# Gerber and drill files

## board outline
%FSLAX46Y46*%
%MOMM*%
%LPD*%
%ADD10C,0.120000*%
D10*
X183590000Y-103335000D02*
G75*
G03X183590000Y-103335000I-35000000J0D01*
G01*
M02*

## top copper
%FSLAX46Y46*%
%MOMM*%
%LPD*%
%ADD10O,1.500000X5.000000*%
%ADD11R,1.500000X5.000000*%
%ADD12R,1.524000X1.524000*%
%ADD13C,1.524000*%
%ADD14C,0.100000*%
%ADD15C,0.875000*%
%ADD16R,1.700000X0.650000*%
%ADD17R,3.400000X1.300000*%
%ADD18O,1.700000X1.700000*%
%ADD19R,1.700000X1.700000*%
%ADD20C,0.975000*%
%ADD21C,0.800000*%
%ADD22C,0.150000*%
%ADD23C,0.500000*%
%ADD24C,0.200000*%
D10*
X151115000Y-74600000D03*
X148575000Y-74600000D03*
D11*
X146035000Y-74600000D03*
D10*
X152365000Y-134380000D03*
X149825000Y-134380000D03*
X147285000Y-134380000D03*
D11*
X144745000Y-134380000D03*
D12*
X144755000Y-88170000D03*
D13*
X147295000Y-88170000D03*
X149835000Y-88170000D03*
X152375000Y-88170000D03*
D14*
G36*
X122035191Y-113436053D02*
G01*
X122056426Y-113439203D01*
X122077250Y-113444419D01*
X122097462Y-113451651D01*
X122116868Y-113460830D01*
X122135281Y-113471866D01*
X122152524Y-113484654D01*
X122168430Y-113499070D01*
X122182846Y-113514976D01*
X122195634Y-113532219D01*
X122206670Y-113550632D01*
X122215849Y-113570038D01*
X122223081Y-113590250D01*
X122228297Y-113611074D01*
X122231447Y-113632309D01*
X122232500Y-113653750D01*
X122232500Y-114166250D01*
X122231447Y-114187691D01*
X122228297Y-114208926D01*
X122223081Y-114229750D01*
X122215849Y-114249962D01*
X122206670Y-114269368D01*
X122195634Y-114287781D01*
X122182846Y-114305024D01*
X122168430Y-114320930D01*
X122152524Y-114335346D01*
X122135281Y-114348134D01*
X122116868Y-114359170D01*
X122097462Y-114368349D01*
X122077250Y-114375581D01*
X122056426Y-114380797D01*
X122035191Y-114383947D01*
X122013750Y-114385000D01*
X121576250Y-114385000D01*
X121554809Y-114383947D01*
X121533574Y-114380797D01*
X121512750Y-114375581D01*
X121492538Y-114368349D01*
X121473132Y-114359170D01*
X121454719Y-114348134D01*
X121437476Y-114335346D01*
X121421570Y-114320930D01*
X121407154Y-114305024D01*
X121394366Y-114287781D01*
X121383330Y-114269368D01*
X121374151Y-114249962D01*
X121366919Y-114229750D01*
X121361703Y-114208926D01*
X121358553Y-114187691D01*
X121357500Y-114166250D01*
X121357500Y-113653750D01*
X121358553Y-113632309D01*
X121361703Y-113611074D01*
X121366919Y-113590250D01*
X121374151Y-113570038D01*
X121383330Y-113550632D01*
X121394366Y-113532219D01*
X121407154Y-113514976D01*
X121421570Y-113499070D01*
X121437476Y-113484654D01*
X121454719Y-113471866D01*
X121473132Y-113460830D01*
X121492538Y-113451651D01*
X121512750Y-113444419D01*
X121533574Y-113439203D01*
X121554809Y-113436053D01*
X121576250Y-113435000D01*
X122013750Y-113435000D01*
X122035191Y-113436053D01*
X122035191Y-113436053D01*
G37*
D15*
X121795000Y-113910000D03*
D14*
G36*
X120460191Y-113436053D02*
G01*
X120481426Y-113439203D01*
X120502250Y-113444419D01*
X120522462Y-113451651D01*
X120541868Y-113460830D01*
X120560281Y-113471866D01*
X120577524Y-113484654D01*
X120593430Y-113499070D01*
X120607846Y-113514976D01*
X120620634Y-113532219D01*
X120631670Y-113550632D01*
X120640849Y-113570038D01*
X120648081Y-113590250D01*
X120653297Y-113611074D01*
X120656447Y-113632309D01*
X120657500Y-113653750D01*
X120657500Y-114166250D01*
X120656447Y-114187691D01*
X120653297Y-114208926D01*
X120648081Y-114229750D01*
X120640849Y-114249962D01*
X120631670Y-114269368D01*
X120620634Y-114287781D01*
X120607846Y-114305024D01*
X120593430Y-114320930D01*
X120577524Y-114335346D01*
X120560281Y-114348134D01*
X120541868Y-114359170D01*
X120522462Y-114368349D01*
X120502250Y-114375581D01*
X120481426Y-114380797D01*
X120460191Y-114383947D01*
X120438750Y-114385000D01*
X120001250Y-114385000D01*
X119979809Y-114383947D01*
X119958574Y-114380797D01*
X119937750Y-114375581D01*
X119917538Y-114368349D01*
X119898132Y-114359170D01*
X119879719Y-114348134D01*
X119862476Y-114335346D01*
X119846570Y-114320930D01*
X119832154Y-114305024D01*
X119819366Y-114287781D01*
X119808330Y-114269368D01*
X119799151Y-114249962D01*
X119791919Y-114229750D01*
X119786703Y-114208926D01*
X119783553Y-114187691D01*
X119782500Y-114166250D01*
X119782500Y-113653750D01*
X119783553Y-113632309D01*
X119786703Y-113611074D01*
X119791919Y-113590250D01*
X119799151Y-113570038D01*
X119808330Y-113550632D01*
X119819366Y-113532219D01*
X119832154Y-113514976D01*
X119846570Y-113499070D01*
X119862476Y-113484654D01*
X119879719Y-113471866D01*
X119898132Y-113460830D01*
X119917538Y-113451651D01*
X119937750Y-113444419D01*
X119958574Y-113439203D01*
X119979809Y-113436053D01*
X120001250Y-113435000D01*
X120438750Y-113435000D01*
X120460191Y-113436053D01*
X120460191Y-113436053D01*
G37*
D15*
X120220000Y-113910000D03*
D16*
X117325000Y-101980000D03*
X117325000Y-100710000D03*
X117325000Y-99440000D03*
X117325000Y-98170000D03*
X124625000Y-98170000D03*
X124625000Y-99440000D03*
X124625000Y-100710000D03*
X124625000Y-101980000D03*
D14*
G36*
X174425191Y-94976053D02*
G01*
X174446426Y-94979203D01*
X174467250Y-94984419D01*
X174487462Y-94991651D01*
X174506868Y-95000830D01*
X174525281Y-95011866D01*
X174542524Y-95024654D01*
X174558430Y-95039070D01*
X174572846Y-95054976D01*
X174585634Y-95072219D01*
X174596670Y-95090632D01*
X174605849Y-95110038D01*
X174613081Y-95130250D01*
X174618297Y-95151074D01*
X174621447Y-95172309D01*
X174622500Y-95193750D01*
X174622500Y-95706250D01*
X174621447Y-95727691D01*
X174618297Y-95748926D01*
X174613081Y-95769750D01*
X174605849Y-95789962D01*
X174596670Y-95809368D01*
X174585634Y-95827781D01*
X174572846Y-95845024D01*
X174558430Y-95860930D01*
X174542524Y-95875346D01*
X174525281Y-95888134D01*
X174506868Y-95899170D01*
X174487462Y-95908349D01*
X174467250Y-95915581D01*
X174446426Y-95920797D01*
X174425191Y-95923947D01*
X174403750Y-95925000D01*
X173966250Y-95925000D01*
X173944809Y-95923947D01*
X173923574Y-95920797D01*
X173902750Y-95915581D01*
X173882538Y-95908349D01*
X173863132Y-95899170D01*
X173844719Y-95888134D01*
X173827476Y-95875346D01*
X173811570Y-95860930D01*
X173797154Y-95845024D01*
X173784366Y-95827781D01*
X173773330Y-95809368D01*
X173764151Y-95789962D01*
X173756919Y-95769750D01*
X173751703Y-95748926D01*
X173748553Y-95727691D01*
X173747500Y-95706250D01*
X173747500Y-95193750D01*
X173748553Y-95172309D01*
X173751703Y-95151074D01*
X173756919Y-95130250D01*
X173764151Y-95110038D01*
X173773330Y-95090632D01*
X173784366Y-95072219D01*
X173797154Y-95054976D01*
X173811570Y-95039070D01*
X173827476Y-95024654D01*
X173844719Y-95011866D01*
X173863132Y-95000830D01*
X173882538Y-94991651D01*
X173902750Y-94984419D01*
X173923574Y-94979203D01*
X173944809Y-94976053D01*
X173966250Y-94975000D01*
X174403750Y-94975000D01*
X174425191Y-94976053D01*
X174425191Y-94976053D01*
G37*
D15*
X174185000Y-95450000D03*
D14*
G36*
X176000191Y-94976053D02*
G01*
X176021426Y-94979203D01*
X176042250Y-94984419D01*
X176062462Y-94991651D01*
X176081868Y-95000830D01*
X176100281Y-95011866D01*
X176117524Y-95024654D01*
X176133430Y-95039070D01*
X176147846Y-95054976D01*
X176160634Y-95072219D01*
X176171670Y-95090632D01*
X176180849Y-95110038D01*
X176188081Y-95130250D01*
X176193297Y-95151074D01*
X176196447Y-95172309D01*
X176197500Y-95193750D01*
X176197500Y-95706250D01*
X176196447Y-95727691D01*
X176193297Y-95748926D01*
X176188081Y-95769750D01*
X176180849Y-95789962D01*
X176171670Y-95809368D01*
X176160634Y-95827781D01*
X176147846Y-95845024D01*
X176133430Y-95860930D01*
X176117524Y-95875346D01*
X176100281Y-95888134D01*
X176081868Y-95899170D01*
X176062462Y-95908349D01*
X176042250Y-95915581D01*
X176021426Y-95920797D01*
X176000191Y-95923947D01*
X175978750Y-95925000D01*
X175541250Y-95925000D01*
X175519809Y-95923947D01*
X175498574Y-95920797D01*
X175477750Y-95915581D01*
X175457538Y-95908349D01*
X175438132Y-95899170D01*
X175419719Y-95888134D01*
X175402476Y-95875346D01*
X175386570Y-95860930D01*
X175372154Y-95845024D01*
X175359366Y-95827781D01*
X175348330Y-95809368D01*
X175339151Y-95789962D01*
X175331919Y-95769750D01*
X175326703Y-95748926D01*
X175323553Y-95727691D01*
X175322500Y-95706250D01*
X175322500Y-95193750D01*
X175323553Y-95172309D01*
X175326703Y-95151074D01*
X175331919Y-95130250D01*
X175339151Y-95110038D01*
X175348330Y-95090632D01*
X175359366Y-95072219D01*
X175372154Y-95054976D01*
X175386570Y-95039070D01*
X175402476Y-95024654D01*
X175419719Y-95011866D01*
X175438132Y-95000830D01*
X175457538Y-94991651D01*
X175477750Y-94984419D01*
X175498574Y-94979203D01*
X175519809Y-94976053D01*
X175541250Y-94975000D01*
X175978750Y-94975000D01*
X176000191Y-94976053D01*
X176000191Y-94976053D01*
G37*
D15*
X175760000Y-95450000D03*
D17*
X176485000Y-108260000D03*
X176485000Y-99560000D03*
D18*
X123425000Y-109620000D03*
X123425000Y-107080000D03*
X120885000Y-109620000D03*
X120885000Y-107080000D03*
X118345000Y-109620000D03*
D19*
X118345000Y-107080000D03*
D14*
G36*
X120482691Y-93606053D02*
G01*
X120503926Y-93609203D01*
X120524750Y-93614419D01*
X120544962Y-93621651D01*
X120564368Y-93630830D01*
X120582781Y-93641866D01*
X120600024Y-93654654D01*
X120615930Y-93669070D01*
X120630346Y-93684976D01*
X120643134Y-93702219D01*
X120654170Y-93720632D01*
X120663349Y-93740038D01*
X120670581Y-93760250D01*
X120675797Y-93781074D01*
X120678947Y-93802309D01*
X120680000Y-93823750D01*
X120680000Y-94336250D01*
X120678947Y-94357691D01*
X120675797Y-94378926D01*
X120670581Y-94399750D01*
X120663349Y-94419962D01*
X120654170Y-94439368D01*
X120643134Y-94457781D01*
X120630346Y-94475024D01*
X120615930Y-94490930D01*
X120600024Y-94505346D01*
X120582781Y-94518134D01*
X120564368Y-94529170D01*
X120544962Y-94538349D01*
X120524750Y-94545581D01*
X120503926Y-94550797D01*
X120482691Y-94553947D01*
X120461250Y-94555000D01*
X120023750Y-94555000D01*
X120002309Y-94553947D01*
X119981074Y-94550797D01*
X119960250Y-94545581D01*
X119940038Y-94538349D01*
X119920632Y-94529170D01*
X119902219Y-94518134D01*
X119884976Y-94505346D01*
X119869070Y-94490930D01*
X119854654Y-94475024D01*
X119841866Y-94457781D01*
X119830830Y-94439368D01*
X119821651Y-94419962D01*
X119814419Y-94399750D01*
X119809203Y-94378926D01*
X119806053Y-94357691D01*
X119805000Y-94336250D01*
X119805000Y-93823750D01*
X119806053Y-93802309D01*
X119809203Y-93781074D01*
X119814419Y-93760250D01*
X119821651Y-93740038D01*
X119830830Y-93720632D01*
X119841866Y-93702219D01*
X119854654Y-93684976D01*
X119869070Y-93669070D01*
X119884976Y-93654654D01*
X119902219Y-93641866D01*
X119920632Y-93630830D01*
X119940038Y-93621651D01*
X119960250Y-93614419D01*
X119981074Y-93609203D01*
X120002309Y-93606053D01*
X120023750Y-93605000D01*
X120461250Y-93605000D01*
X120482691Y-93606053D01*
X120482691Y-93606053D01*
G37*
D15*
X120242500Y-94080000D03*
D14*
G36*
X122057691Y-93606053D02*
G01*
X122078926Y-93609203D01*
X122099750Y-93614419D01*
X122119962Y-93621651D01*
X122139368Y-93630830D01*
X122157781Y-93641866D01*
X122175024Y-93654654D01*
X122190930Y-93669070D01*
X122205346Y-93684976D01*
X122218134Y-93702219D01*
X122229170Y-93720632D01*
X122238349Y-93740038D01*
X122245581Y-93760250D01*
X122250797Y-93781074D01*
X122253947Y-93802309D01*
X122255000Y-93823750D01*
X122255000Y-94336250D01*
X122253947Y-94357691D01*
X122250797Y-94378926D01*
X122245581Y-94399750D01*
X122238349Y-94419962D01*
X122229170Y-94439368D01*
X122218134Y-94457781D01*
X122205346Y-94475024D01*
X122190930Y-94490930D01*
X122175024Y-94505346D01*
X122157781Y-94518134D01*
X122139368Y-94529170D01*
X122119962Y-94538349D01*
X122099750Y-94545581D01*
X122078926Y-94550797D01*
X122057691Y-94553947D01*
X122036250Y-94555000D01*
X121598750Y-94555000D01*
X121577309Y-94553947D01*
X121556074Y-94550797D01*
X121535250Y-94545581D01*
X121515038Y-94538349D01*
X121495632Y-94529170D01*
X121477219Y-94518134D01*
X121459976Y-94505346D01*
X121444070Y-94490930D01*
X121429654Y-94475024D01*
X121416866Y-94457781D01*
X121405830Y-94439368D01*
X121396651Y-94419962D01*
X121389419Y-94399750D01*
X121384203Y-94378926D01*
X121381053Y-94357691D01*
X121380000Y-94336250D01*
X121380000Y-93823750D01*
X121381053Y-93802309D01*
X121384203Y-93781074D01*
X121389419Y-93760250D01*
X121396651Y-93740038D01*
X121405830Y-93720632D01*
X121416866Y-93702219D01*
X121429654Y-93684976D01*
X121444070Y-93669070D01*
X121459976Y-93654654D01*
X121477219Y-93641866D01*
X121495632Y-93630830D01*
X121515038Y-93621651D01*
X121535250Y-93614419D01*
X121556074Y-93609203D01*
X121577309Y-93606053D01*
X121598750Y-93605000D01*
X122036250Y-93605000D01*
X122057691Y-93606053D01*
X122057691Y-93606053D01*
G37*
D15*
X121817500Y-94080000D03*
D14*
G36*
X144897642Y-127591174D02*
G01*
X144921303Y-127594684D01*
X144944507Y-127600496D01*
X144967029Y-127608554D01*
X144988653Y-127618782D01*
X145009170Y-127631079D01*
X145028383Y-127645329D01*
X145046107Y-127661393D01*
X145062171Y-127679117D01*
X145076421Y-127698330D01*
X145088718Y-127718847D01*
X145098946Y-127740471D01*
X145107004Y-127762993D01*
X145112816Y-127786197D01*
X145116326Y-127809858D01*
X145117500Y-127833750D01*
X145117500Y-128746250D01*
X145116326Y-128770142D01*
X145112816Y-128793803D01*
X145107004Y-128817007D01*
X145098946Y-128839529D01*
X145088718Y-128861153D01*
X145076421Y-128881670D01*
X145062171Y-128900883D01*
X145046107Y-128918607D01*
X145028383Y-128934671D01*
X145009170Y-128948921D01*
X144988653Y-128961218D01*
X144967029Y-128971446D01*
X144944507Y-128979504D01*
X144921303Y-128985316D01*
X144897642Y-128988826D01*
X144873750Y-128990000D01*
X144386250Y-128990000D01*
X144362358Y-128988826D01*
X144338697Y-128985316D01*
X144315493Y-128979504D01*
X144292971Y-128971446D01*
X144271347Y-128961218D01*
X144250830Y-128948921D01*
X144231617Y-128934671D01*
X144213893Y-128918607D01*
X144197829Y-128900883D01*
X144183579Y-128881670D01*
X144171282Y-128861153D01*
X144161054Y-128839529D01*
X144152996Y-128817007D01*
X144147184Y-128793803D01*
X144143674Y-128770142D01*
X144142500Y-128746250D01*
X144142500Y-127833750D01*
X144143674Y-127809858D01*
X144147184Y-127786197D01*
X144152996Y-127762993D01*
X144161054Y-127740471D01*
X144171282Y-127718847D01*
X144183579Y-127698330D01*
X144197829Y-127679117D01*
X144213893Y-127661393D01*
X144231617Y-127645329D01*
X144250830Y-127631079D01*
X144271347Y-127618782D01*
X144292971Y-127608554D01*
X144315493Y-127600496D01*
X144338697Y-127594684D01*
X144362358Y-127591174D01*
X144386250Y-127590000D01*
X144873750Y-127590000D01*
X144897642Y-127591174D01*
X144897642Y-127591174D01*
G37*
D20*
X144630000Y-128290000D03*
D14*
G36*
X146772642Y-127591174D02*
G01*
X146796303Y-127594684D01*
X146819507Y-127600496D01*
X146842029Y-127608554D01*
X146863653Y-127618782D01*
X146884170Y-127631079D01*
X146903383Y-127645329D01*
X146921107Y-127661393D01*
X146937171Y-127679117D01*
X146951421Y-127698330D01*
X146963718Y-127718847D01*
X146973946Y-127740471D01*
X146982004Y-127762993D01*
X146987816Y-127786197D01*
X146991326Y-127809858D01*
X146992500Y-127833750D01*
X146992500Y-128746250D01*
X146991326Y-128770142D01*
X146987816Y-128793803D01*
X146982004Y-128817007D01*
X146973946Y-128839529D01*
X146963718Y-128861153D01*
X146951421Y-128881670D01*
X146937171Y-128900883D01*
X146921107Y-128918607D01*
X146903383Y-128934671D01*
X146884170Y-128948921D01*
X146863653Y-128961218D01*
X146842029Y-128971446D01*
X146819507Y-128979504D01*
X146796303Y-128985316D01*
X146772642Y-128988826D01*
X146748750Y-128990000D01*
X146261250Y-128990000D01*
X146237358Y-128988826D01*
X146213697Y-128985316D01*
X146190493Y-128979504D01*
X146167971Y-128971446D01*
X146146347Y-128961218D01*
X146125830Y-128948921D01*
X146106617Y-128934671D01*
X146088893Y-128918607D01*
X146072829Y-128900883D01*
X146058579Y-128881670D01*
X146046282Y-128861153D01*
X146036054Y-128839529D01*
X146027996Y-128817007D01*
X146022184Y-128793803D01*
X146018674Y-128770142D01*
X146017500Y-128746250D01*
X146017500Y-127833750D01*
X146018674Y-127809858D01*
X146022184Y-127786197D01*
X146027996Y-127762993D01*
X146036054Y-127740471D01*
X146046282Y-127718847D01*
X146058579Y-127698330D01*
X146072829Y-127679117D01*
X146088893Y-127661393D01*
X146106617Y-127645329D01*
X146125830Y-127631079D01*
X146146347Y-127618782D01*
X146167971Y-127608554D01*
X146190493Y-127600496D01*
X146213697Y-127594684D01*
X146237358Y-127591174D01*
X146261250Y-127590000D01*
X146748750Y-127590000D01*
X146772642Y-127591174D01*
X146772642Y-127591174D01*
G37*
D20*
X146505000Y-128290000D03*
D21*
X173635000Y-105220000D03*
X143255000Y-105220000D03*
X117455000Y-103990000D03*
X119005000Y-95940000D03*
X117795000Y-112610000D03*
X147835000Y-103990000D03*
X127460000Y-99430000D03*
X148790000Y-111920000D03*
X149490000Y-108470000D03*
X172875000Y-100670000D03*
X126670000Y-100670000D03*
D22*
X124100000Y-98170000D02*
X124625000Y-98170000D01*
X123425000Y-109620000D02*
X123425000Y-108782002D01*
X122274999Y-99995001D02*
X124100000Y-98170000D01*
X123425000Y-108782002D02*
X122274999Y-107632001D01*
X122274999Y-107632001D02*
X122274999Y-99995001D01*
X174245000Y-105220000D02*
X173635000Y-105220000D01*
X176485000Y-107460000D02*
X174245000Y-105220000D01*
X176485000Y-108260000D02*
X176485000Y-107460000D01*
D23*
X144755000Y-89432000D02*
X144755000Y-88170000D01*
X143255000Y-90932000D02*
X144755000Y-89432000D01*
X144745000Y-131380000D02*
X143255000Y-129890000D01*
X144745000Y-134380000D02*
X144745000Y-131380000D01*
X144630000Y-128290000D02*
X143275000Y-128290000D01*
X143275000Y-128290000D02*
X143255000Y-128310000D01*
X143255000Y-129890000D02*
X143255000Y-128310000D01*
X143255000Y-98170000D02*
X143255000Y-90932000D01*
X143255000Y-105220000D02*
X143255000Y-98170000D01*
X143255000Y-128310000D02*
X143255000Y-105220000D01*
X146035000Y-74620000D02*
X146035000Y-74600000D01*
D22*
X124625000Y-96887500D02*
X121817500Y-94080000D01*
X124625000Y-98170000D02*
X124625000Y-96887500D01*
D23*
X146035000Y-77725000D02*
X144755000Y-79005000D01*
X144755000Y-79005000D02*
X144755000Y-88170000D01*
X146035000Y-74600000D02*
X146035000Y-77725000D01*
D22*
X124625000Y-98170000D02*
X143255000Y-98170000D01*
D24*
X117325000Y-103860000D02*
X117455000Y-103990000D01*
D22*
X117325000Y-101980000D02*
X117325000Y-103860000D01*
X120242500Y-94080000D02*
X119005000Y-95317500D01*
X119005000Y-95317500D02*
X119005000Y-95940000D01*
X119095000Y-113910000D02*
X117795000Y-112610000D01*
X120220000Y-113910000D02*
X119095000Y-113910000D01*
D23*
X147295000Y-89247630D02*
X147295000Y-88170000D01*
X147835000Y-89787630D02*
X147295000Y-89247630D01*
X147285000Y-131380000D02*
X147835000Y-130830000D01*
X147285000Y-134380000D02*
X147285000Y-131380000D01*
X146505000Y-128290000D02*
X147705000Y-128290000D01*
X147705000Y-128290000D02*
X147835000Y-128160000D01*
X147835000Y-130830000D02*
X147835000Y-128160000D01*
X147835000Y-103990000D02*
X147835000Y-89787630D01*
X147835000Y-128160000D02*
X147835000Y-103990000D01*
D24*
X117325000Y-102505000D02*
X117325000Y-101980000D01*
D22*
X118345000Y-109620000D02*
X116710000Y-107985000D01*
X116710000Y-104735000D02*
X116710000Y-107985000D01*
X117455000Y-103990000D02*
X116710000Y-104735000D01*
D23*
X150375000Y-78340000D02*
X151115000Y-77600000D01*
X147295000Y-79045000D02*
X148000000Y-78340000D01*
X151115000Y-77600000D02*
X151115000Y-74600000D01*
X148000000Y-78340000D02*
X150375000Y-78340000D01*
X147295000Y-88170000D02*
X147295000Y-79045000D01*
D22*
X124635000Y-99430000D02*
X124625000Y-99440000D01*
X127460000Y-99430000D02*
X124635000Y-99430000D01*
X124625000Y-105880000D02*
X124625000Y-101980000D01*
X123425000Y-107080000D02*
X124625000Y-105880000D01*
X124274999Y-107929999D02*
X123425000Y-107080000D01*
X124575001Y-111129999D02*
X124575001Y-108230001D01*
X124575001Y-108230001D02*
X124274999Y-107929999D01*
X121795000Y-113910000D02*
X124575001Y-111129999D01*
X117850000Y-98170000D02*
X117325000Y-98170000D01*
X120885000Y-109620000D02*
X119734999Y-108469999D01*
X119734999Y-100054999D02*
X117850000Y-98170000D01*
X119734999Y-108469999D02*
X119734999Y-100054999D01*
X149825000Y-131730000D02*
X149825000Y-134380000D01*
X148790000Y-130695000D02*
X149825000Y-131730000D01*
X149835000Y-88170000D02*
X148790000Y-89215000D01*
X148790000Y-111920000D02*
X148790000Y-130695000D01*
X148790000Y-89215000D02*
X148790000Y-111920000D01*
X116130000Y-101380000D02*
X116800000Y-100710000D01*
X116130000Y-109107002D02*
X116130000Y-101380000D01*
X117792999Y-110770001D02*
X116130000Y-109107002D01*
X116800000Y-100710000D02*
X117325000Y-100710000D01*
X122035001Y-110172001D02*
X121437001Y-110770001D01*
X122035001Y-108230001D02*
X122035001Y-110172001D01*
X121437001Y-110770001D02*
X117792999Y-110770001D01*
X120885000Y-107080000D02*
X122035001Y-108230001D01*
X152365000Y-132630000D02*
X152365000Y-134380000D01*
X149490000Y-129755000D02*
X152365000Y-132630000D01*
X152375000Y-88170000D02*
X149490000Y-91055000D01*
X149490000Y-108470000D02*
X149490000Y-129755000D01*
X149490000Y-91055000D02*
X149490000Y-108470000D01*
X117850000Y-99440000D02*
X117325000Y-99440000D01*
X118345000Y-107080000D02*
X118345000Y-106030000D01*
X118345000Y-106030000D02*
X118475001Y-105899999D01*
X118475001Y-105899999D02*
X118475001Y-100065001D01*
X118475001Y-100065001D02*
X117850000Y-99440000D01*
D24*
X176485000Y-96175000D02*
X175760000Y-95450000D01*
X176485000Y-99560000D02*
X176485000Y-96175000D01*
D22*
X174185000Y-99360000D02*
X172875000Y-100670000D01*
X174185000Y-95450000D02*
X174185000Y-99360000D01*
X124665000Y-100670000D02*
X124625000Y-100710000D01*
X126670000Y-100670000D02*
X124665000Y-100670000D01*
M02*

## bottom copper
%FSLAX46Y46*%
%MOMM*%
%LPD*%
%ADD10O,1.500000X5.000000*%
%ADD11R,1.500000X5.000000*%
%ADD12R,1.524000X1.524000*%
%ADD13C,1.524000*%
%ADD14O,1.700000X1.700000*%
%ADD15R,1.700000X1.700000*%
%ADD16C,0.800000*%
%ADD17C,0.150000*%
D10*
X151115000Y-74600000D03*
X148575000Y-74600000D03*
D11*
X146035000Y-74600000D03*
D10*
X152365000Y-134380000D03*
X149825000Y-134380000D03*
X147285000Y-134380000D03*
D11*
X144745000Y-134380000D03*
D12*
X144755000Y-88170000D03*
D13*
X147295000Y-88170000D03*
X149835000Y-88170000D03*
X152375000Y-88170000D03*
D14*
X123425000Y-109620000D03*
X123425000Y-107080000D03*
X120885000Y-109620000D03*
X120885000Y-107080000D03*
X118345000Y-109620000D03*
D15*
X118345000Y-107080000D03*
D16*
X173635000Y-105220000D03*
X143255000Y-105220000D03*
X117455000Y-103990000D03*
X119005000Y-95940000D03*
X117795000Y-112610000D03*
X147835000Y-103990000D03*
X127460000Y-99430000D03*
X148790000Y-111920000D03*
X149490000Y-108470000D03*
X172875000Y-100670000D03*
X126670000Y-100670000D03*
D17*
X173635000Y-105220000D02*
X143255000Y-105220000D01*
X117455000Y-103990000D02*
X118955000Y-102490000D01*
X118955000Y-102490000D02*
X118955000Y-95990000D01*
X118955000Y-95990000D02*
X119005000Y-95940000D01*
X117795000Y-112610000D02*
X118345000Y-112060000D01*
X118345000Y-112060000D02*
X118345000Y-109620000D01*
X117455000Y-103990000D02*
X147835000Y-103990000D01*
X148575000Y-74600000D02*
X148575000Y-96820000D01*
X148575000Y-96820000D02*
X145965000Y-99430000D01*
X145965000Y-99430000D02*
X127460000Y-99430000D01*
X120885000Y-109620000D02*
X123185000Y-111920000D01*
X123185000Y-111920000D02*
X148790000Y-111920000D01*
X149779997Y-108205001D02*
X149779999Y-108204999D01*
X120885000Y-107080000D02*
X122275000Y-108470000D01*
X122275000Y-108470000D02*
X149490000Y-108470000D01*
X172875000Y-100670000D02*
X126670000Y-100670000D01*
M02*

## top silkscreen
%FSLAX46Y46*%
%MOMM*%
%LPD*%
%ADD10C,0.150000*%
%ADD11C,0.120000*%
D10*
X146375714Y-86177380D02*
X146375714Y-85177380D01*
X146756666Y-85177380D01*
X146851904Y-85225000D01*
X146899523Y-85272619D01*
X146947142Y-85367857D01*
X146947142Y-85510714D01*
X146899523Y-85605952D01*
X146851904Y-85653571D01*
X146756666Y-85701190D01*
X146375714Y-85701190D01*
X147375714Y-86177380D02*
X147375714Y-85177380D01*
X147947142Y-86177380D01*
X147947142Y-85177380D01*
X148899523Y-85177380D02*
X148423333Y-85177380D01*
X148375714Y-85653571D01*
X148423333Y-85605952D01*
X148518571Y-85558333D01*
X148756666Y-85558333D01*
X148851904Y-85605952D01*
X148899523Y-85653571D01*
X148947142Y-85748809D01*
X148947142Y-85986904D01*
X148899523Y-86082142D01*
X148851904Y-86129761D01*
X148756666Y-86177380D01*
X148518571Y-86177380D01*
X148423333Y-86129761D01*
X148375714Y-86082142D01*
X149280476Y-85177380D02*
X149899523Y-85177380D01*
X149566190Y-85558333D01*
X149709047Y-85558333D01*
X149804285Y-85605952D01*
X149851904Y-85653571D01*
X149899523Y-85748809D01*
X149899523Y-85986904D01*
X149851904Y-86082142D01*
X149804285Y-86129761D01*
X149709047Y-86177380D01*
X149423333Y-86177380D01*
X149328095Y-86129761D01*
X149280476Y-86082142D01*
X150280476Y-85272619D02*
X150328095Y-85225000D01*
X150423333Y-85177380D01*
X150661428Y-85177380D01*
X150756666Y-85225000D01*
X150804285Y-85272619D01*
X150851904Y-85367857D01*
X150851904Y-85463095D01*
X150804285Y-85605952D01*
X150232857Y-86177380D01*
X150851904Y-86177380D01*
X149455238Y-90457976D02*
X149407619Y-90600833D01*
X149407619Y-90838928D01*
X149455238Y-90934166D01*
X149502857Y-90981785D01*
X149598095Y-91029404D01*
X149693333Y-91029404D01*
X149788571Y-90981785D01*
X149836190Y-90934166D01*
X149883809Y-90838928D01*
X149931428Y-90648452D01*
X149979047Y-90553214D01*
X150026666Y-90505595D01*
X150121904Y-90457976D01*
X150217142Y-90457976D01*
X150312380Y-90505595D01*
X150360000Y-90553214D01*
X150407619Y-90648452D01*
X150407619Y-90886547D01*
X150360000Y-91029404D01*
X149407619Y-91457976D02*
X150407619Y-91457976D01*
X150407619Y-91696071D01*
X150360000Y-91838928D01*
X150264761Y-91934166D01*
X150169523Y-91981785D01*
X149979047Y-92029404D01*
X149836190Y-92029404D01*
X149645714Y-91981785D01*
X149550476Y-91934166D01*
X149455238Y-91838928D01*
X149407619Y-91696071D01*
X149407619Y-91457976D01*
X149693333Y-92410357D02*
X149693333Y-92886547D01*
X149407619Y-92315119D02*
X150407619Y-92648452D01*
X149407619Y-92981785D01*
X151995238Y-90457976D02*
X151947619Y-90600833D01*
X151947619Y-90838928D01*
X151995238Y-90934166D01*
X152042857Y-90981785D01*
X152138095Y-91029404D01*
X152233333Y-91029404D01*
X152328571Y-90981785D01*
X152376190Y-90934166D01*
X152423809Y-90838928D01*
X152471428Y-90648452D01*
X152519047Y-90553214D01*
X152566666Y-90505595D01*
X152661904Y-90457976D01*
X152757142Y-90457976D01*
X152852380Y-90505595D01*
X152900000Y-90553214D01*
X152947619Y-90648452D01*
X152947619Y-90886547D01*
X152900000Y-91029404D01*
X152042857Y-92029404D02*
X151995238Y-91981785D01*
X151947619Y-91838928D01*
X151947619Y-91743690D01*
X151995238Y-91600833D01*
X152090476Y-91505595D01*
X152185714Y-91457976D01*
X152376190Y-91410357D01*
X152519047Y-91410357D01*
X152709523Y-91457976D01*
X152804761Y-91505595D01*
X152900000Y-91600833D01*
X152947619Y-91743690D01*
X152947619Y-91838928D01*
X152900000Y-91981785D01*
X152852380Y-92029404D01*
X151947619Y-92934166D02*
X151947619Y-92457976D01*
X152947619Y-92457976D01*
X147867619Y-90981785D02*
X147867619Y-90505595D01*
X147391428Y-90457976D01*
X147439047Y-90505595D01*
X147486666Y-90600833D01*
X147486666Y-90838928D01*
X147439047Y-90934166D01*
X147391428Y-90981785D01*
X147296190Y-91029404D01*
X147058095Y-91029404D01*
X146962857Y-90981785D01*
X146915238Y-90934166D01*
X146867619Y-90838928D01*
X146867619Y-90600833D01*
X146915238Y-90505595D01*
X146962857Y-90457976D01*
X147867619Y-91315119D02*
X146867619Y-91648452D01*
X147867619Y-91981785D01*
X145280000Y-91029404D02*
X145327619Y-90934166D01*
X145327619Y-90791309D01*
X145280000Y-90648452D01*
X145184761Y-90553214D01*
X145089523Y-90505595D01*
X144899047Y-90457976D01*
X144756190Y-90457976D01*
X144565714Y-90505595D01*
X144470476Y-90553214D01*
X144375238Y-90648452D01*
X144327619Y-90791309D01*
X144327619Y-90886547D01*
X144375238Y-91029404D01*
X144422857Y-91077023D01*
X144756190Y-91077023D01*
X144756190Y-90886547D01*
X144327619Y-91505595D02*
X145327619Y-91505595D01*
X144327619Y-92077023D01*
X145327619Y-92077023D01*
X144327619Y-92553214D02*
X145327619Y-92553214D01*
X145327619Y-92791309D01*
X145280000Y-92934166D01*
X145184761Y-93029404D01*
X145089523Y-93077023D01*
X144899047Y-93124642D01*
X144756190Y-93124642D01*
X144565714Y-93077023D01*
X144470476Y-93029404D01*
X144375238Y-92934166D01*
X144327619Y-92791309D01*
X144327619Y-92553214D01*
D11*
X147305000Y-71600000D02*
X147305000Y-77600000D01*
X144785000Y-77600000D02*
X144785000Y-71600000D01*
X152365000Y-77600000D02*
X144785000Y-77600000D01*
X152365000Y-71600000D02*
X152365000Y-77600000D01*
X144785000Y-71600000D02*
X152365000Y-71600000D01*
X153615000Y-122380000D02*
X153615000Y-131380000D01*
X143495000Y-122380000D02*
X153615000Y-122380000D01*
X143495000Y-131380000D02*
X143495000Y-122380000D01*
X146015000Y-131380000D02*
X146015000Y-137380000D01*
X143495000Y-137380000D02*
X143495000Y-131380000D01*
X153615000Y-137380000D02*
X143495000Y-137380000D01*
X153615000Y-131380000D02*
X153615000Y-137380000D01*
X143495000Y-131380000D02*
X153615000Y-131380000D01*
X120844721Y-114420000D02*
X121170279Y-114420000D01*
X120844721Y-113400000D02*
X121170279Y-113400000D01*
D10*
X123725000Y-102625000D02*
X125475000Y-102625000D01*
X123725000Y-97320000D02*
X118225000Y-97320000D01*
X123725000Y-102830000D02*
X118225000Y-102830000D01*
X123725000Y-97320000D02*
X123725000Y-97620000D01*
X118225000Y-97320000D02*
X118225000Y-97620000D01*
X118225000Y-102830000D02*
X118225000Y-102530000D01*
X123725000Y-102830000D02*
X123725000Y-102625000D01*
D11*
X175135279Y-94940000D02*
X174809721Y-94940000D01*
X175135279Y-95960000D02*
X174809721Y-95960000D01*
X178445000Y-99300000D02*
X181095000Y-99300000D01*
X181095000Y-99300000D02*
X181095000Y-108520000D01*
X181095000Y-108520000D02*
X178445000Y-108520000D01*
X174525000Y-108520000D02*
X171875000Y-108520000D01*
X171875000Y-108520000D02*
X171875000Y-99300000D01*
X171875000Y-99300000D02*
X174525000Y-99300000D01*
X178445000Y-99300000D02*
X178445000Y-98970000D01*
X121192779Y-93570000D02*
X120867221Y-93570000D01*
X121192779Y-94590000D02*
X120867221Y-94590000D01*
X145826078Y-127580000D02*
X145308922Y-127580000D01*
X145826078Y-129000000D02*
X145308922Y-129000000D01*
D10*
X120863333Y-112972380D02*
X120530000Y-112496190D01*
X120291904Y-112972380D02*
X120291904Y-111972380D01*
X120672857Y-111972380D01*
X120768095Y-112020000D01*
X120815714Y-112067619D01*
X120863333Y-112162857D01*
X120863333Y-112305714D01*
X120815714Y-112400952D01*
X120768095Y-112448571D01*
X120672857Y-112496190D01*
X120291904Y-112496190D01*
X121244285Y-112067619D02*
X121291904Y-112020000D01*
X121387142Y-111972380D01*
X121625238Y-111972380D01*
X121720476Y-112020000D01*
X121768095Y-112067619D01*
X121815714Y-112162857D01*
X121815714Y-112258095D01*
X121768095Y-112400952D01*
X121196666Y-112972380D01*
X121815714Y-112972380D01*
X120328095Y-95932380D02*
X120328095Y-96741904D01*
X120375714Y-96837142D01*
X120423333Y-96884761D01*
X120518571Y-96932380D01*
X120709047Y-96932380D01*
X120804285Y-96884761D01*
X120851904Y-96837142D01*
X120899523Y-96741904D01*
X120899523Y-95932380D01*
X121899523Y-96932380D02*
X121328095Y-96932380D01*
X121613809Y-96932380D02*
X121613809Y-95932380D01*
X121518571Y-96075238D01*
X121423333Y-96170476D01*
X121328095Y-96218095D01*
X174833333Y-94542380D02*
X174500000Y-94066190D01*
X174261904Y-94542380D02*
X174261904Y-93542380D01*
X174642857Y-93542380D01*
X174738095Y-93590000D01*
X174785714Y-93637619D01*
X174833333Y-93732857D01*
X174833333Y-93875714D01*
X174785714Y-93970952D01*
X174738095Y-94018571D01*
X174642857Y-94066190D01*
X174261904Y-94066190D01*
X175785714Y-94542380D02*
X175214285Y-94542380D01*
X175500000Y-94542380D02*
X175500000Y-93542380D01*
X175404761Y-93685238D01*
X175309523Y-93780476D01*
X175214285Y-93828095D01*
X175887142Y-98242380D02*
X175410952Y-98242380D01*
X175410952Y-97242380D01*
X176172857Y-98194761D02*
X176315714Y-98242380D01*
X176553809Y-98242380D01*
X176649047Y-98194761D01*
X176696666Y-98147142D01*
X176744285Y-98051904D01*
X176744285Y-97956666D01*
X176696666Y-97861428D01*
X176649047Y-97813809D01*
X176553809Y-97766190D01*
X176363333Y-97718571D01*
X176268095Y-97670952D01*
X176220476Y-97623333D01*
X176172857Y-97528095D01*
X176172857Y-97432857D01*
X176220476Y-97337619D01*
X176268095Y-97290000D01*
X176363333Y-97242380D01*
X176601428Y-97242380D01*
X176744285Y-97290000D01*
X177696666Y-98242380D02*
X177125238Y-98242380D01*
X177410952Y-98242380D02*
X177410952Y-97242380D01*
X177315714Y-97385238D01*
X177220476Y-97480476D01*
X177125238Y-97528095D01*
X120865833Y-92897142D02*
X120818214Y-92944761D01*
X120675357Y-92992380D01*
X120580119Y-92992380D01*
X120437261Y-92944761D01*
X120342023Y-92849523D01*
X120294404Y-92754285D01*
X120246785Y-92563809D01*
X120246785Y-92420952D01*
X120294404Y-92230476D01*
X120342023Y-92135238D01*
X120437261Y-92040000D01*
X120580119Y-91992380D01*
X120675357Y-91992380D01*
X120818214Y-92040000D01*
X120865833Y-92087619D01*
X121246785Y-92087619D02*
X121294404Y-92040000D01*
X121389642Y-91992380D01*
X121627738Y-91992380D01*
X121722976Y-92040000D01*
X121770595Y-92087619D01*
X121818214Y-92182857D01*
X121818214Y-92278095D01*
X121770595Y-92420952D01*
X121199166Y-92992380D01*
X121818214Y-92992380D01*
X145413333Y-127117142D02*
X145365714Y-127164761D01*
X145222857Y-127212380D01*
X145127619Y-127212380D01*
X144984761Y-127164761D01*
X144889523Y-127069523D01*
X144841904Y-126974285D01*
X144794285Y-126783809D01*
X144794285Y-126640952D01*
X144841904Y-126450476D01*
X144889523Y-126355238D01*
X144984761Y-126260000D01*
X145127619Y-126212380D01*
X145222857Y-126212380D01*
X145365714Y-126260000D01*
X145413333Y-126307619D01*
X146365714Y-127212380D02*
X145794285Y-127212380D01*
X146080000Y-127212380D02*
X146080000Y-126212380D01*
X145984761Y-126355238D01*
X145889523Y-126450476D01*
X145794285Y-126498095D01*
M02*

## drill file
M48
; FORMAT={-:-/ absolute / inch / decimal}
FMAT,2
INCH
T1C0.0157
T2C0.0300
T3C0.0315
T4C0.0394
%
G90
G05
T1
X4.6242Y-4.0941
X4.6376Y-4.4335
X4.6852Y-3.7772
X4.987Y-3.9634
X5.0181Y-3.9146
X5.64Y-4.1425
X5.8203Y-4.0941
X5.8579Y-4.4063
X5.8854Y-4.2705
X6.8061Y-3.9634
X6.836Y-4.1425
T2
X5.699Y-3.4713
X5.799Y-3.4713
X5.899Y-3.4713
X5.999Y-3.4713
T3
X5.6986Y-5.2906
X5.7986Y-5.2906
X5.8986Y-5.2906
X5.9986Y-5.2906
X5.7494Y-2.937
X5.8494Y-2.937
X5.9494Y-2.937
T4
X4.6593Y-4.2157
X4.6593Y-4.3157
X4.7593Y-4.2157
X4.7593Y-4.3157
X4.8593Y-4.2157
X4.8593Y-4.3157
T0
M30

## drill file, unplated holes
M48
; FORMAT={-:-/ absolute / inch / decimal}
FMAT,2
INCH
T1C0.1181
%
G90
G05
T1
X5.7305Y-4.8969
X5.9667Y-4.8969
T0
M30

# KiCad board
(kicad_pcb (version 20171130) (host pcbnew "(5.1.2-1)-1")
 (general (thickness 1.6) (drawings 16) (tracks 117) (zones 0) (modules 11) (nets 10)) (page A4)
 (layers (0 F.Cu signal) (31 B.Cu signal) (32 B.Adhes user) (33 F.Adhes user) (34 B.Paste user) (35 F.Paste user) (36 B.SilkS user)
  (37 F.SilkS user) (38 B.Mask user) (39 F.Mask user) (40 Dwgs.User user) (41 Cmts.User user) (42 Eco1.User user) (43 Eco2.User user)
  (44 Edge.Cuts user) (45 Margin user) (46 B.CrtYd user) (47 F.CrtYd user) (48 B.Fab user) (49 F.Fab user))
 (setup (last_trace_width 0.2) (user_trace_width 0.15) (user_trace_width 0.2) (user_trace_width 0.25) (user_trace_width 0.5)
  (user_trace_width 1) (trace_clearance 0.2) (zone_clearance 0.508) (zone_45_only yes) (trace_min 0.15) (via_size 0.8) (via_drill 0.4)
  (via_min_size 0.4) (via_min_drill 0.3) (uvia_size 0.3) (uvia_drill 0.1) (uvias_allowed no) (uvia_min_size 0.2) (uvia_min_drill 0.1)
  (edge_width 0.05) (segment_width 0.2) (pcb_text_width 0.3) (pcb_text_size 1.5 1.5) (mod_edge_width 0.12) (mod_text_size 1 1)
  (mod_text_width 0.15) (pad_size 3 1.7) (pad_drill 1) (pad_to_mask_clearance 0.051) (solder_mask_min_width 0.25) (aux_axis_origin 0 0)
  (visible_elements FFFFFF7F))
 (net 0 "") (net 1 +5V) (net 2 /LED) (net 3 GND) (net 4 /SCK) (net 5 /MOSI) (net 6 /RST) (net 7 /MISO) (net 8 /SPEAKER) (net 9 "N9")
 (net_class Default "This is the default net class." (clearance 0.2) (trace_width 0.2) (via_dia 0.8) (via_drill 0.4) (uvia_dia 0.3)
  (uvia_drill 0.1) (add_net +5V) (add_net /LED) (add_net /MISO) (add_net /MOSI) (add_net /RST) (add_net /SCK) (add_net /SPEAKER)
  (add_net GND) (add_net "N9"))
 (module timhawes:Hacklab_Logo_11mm (layer B.Cu) (at 174.32 101.97 180)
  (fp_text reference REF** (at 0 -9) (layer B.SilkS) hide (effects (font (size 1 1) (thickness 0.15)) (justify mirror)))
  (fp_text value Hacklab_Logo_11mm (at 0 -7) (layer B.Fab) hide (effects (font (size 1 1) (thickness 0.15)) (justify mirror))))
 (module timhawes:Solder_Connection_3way (layer F.Cu) (at 148.575 74.6)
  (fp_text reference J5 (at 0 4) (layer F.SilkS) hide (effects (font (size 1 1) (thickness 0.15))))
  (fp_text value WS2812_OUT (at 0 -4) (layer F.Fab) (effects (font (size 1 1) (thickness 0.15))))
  (fp_line (start -1.27 -3) (end -1.27 3) (layer F.SilkS) (width 0.12))
  (fp_line (start -3.79 3) (end -3.79 -3) (layer F.SilkS) (width 0.12))
  (fp_line (start 3.79 3) (end -3.79 3) (layer F.SilkS) (width 0.12))
  (fp_line (start 3.79 -3) (end 3.79 3) (layer F.SilkS) (width 0.12))
  (fp_line (start -3.79 -3) (end 3.79 -3) (layer F.SilkS) (width 0.12))
  (pad 3 thru_hole oval (at 2.54 0) (size 1.5 5) (drill 0.8) (layers *.Cu *.Mask) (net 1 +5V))
  (pad 2 thru_hole oval (at 0 0) (size 1.5 5) (drill 0.8) (layers *.Cu *.Mask) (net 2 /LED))
  (pad 1 thru_hole rect (at -2.54 0) (size 1.5 5) (drill 0.8) (layers *.Cu *.Mask) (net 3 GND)))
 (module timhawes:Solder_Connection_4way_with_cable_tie (layer F.Cu) (at 148.555 134.38)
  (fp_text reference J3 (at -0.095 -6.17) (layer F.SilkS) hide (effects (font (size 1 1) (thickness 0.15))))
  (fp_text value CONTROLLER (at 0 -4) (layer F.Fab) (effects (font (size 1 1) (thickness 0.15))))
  (fp_line (start 5.06 -12) (end 5.06 -3) (layer F.SilkS) (width 0.12))
  (fp_line (start -5.06 -12) (end 5.06 -12) (layer F.SilkS) (width 0.12))
  (fp_line (start -5.06 -3) (end -5.06 -12) (layer F.SilkS) (width 0.12))
  (fp_line (start -2.54 -3) (end -2.54 3) (layer F.SilkS) (width 0.12))
  (fp_line (start -5.06 3) (end -5.06 -3) (layer F.SilkS) (width 0.12))
  (fp_line (start 5.06 3) (end -5.06 3) (layer F.SilkS) (width 0.12))
  (fp_line (start 5.06 -3) (end 5.06 3) (layer F.SilkS) (width 0.12))
  (fp_line (start -5.06 -3) (end 5.06 -3) (layer F.SilkS) (width 0.12))
  (pad "" np_thru_hole circle (at 3 -10) (size 3 3) (drill 3) (layers *.Cu *.Mask))
  (pad "" np_thru_hole circle (at -3 -10) (size 3 3) (drill 3) (layers *.Cu *.Mask))
  (pad 4 thru_hole oval (at 3.81 0) (size 1.5 5) (drill 0.8) (layers *.Cu *.Mask) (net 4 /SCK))
  (pad 3 thru_hole oval (at 1.27 0) (size 1.5 5) (drill 0.8) (layers *.Cu *.Mask) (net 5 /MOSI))
  (pad 2 thru_hole oval (at -1.27 0) (size 1.5 5) (drill 0.8) (layers *.Cu *.Mask) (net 1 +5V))
  (pad 1 thru_hole rect (at -3.81 0) (size 1.5 5) (drill 0.8) (layers *.Cu *.Mask) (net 3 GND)))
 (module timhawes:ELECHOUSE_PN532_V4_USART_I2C (layer B.Cu) (at 148.545 107.99)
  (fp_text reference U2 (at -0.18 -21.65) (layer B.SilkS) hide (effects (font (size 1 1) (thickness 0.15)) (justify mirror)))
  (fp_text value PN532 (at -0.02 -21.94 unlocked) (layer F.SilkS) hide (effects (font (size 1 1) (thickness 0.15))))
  (pad 1 thru_hole rect (at -3.79 -19.82) (size 1.524 1.524) (drill 0.762) (layers *.Cu *.Mask) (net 3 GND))
  (pad 2 thru_hole circle (at -1.25 -19.82) (size 1.524 1.524) (drill 0.762) (layers *.Cu *.Mask) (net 1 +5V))
  (pad 3 thru_hole circle (at 1.29 -19.82) (size 1.524 1.524) (drill 0.762) (layers *.Cu *.Mask) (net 5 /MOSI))
  (pad 4 thru_hole circle (at 3.83 -19.82) (size 1.524 1.524) (drill 0.762) (layers *.Cu *.Mask) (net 4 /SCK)))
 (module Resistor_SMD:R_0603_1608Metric (layer F.Cu) (at 121.0075 113.91)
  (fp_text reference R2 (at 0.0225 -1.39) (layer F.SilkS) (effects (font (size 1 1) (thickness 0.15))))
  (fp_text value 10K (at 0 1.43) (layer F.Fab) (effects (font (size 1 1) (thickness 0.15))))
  (fp_line (start -0.162779 0.51) (end 0.162779 0.51) (layer F.SilkS) (width 0.12))
  (fp_line (start -0.162779 -0.51) (end 0.162779 -0.51) (layer F.SilkS) (width 0.12))
  (pad 2 smd roundrect (at 0.7875 0) (size 0.875 0.95) (layers F.Cu F.Paste F.Mask) (roundrect_rratio 0.25) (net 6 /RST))
  (pad 1 smd roundrect (at -0.7875 0) (size 0.875 0.95) (layers F.Cu F.Paste F.Mask) (roundrect_rratio 0.25) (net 1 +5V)))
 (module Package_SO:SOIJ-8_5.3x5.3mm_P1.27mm (layer F.Cu) (at 120.975 100.075 180)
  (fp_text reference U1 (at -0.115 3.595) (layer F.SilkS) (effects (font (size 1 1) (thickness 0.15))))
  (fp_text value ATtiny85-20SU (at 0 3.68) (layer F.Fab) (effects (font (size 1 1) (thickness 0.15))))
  (fp_line (start -2.75 -2.55) (end -4.5 -2.55) (layer F.SilkS) (width 0.15))
  (fp_line (start -2.75 2.755) (end 2.75 2.755) (layer F.SilkS) (width 0.15))
  (fp_line (start -2.75 -2.755) (end 2.75 -2.755) (layer F.SilkS) (width 0.15))
  (fp_line (start -2.75 2.755) (end -2.75 2.455) (layer F.SilkS) (width 0.15))
  (fp_line (start 2.75 2.755) (end 2.75 2.455) (layer F.SilkS) (width 0.15))
  (fp_line (start 2.75 -2.755) (end 2.75 -2.455) (layer F.SilkS) (width 0.15))
  (fp_line (start -2.75 -2.755) (end -2.75 -2.55) (layer F.SilkS) (width 0.15))
  (pad 8 smd rect (at 3.65 -1.905 180) (size 1.7 0.65) (layers F.Cu F.Paste F.Mask) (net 1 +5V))
  (pad 7 smd rect (at 3.65 -0.635 180) (size 1.7 0.65) (layers F.Cu F.Paste F.Mask) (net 4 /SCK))
  (pad 6 smd rect (at 3.65 0.635 180) (size 1.7 0.65) (layers F.Cu F.Paste F.Mask) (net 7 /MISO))
  (pad 5 smd rect (at 3.65 1.905 180) (size 1.7 0.65) (layers F.Cu F.Paste F.Mask) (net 5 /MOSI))
  (pad 4 smd rect (at -3.65 1.905 180) (size 1.7 0.65) (layers F.Cu F.Paste F.Mask) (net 3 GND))
  (pad 3 smd rect (at -3.65 0.635 180) (size 1.7 0.65) (layers F.Cu F.Paste F.Mask) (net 2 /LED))
  (pad 2 smd rect (at -3.65 -0.635 180) (size 1.7 0.65) (layers F.Cu F.Paste F.Mask) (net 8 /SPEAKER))
  (pad 1 smd rect (at -3.65 -1.905 180) (size 1.7 0.65) (layers F.Cu F.Paste F.Mask) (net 6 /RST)))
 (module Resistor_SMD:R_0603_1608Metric (layer F.Cu) (at 174.9725 95.45 180)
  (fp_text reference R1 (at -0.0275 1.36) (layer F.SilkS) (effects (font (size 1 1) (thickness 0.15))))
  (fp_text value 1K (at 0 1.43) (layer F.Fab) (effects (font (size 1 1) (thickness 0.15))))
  (fp_line (start -0.162779 0.51) (end 0.162779 0.51) (layer F.SilkS) (width 0.12))
  (fp_line (start -0.162779 -0.51) (end 0.162779 -0.51) (layer F.SilkS) (width 0.12))
  (pad 2 smd roundrect (at 0.7875 0 180) (size 0.875 0.95) (layers F.Cu F.Paste F.Mask) (roundrect_rratio 0.25) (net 8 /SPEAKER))
  (pad 1 smd roundrect (at -0.7875 0 180) (size 0.875 0.95) (layers F.Cu F.Paste F.Mask) (roundrect_rratio 0.25) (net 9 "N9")))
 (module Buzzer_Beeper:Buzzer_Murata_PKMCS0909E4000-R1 (layer F.Cu) (at 176.485 103.91 270)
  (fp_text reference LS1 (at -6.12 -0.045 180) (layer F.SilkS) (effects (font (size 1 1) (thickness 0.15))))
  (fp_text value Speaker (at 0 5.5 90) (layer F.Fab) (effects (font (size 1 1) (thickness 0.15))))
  (fp_line (start -4.61 -1.96) (end -4.61 -4.61) (layer F.SilkS) (width 0.12))
  (fp_line (start -4.61 -4.61) (end 4.61 -4.61) (layer F.SilkS) (width 0.12))
  (fp_line (start 4.61 -4.61) (end 4.61 -1.96) (layer F.SilkS) (width 0.12))
  (fp_line (start 4.61 1.96) (end 4.61 4.61) (layer F.SilkS) (width 0.12))
  (fp_line (start 4.61 4.61) (end -4.61 4.61) (layer F.SilkS) (width 0.12))
  (fp_line (start -4.61 4.61) (end -4.61 1.96) (layer F.SilkS) (width 0.12))
  (fp_line (start -4.61 -1.96) (end -4.94 -1.96) (layer F.SilkS) (width 0.12))
  (pad 2 smd rect (at 4.35 0 270) (size 1.3 3.4) (layers F.Cu F.Paste F.Mask) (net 3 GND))
  (pad 1 smd rect (at -4.35 0 270) (size 1.3 3.4) (layers F.Cu F.Paste F.Mask) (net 9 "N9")))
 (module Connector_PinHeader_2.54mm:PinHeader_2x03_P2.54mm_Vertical (layer B.Cu) (at 118.345 107.08 270)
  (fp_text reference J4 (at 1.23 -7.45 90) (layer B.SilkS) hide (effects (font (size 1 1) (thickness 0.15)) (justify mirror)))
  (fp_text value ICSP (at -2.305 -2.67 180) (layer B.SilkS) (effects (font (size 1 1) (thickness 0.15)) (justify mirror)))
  (pad 6 thru_hole oval (at 2.54 -5.08 270) (size 1.7 1.7) (drill 1) (layers *.Cu *.Mask) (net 3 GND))
  (pad 5 thru_hole oval (at 0 -5.08 270) (size 1.7 1.7) (drill 1) (layers *.Cu *.Mask) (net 6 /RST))
  (pad 4 thru_hole oval (at 2.54 -2.54 270) (size 1.7 1.7) (drill 1) (layers *.Cu *.Mask) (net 5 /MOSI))
  (pad 3 thru_hole oval (at 0 -2.54 270) (size 1.7 1.7) (drill 1) (layers *.Cu *.Mask) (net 4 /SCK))
  (pad 2 thru_hole oval (at 2.54 0 270) (size 1.7 1.7) (drill 1) (layers *.Cu *.Mask) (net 1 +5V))
  (pad 1 thru_hole rect (at 0 0 270) (size 1.7 1.7) (drill 1) (layers *.Cu *.Mask) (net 7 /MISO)))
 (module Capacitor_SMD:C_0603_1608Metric (layer F.Cu) (at 121.03 94.08 180)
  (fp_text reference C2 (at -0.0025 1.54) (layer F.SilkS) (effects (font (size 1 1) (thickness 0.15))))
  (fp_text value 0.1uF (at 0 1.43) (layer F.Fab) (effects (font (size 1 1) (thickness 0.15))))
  (fp_line (start -0.162779 0.51) (end 0.162779 0.51) (layer F.SilkS) (width 0.12))
  (fp_line (start -0.162779 -0.51) (end 0.162779 -0.51) (layer F.SilkS) (width 0.12))
  (pad 2 smd roundrect (at 0.7875 0 180) (size 0.875 0.95) (layers F.Cu F.Paste F.Mask) (roundrect_rratio 0.25) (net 1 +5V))
  (pad 1 smd roundrect (at -0.7875 0 180) (size 0.875 0.95) (layers F.Cu F.Paste F.Mask) (roundrect_rratio 0.25) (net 3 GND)))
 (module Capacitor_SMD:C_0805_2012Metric (layer F.Cu) (at 145.5675 128.29 180)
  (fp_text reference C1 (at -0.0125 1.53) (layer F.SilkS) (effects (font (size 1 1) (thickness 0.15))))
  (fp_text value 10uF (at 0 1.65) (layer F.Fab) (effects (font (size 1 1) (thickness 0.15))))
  (fp_line (start -0.258578 0.71) (end 0.258578 0.71) (layer F.SilkS) (width 0.12))
  (fp_line (start -0.258578 -0.71) (end 0.258578 -0.71) (layer F.SilkS) (width 0.12))
  (pad 2 smd roundrect (at 0.9375 0 180) (size 0.975 1.4) (layers F.Cu F.Paste F.Mask) (roundrect_rratio 0.25) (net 3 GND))
  (pad 1 smd roundrect (at -0.9375 0 180) (size 0.975 1.4) (layers F.Cu F.Paste F.Mask) (roundrect_rratio 0.25) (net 1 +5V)))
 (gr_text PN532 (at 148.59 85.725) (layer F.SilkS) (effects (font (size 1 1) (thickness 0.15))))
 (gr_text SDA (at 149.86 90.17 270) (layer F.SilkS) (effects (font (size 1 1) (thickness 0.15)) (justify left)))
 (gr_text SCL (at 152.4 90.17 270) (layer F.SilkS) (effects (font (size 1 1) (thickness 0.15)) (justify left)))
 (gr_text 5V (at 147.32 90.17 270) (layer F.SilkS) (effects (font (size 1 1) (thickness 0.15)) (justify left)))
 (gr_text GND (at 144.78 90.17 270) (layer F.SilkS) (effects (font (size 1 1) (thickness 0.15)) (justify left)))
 (gr_circle (center 148.59 103.335) (end 113.59 103.335) (layer Edge.Cuts) (width 0.12))
 (segment (start 124.1 98.17) (end 124.625 98.17) (width 0.15) (layer F.Cu) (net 3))
 (segment (start 123.425 109.62) (end 123.425 108.782002) (width 0.15) (layer F.Cu) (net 3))
 (segment (start 122.274999 99.995001) (end 124.1 98.17) (width 0.15) (layer F.Cu) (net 3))
 (segment (start 123.425 108.782002) (end 122.274999 107.632001) (width 0.15) (layer F.Cu) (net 3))
 (segment (start 122.274999 107.632001) (end 122.274999 99.995001) (width 0.15) (layer F.Cu) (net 3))
 (via (at 173.635 105.22) (size 0.8) (drill 0.4) (layers F.Cu B.Cu) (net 3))
 (segment (start 174.245 105.22) (end 173.635 105.22) (width 0.15) (layer F.Cu) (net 3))
 (segment (start 176.485 107.46) (end 174.245 105.22) (width 0.15) (layer F.Cu) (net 3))
 (segment (start 176.485 108.26) (end 176.485 107.46) (width 0.15) (layer F.Cu) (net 3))
 (segment (start 144.755 89.432) (end 144.755 88.17) (width 0.5) (layer F.Cu) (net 3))
 (segment (start 143.255 90.932) (end 144.755 89.432) (width 0.5) (layer F.Cu) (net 3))
 (segment (start 144.745 131.38) (end 143.255 129.89) (width 0.5) (layer F.Cu) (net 3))
 (segment (start 144.745 134.38) (end 144.745 131.38) (width 0.5) (layer F.Cu) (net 3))
 (segment (start 144.63 128.29) (end 143.275 128.29) (width 0.5) (layer F.Cu) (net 3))
 (segment (start 143.275 128.29) (end 143.255 128.31) (width 0.5) (layer F.Cu) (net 3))
 (segment (start 143.255 129.89) (end 143.255 128.31) (width 0.5) (layer F.Cu) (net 3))
 (segment (start 143.255 98.17) (end 143.255 90.932) (width 0.5) (layer F.Cu) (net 3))
 (via (at 143.255 105.22) (size 0.8) (drill 0.4) (layers F.Cu B.Cu) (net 3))
 (segment (start 143.255 105.22) (end 143.255 98.17) (width 0.5) (layer F.Cu) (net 3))
 (segment (start 173.635 105.22) (end 143.255 105.22) (width 0.15) (layer B.Cu) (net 3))
 (segment (start 143.255 128.31) (end 143.255 105.22) (width 0.5) (layer F.Cu) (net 3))
 (segment (start 146.035 74.62) (end 146.035 74.6) (width 0.5) (layer F.Cu) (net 3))
 (segment (start 124.625 96.8875) (end 121.8175 94.08) (width 0.15) (layer F.Cu) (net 3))
 (segment (start 124.625 98.17) (end 124.625 96.8875) (width 0.15) (layer F.Cu) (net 3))
 (segment (start 146.035 77.725) (end 144.755 79.005) (width 0.5) (layer F.Cu) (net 3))
 (segment (start 144.755 79.005) (end 144.755 88.17) (width 0.5) (layer F.Cu) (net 3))
 (segment (start 146.035 74.6) (end 146.035 77.725) (width 0.5) (layer F.Cu) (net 3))
 (segment (start 124.625 98.17) (end 143.255 98.17) (width 0.15) (layer F.Cu) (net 3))
 (via (at 117.455 103.99) (size 0.8) (drill 0.4) (layers F.Cu B.Cu) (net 1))
 (segment (start 117.325 103.86) (end 117.455 103.99) (width 0.2) (layer F.Cu) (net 1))
 (segment (start 117.325 101.98) (end 117.325 103.86) (width 0.15) (layer F.Cu) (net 1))
 (segment (start 117.455 103.99) (end 118.955 102.49) (width 0.15) (layer B.Cu) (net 1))
 (segment (start 120.2425 94.08) (end 119.005 95.3175) (width 0.15) (layer F.Cu) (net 1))
 (segment (start 119.005 95.3175) (end 119.005 95.94) (width 0.15) (layer F.Cu) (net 1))
 (segment (start 118.955 102.49) (end 118.955 95.99) (width 0.15) (layer B.Cu) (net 1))
 (segment (start 118.955 95.99) (end 119.005 95.94) (width 0.15) (layer B.Cu) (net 1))
 (via (at 119.005 95.94) (size 0.8) (drill 0.4) (layers F.Cu B.Cu) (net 1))
 (segment (start 119.095 113.91) (end 117.795 112.61) (width 0.15) (layer F.Cu) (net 1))
 (segment (start 117.795 112.61) (end 118.345 112.06) (width 0.15) (layer B.Cu) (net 1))
 (segment (start 118.345 112.06) (end 118.345 109.62) (width 0.15) (layer B.Cu) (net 1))
 (segment (start 120.22 113.91) (end 119.095 113.91) (width 0.15) (layer F.Cu) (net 1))
 (via (at 117.795 112.61) (size 0.8) (drill 0.4) (layers F.Cu B.Cu) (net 1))
 (segment (start 147.295 89.24763) (end 147.295 88.17) (width 0.5) (layer F.Cu) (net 1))
 (segment (start 147.835 89.78763) (end 147.295 89.24763) (width 0.5) (layer F.Cu) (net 1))
 (segment (start 147.285 131.38) (end 147.835 130.83) (width 0.5) (layer F.Cu) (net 1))
 (segment (start 147.285 134.38) (end 147.285 131.38) (width 0.5) (layer F.Cu) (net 1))
 (segment (start 146.505 128.29) (end 147.705 128.29) (width 0.5) (layer F.Cu) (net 1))
 (segment (start 147.705 128.29) (end 147.835 128.16) (width 0.5) (layer F.Cu) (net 1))
 (segment (start 147.835 130.83) (end 147.835 128.16) (width 0.5) (layer F.Cu) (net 1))
 (via (at 147.835 103.99) (size 0.8) (drill 0.4) (layers F.Cu B.Cu) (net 1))
 (segment (start 147.835 103.99) (end 147.835 89.78763) (width 0.5) (layer F.Cu) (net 1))
 (segment (start 147.835 128.16) (end 147.835 103.99) (width 0.5) (layer F.Cu) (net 1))
 (segment (start 117.325 102.505) (end 117.325 101.98) (width 0.2) (layer F.Cu) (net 1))
 (segment (start 118.345 109.62) (end 116.71 107.985) (width 0.15) (layer F.Cu) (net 1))
 (segment (start 116.71 104.735) (end 116.71 107.985) (width 0.15) (layer F.Cu) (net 1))
 (segment (start 117.455 103.99) (end 116.71 104.735) (width 0.15) (layer F.Cu) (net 1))
 (segment (start 150.375 78.34) (end 151.115 77.6) (width 0.5) (layer F.Cu) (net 1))
 (segment (start 147.295 79.045) (end 148 78.34) (width 0.5) (layer F.Cu) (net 1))
 (segment (start 151.115 77.6) (end 151.115 74.6) (width 0.5) (layer F.Cu) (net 1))
 (segment (start 148 78.34) (end 150.375 78.34) (width 0.5) (layer F.Cu) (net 1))
 (segment (start 147.295 88.17) (end 147.295 79.045) (width 0.5) (layer F.Cu) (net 1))
 (segment (start 117.455 103.99) (end 147.835 103.99) (width 0.15) (layer B.Cu) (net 1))
 (segment (start 148.575 74.6) (end 148.575 96.82) (width 0.15) (layer B.Cu) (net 2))
 (segment (start 148.575 96.82) (end 145.965 99.43) (width 0.15) (layer B.Cu) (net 2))
 (via (at 127.46 99.43) (size 0.8) (drill 0.4) (layers F.Cu B.Cu) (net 2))
 (segment (start 145.965 99.43) (end 127.46 99.43) (width 0.15) (layer B.Cu) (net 2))
 (segment (start 124.635 99.43) (end 124.625 99.44) (width 0.15) (layer F.Cu) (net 2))
 (segment (start 127.46 99.43) (end 124.635 99.43) (width 0.15) (layer F.Cu) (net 2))
 (segment (start 124.625 105.88) (end 124.625 101.98) (width 0.15) (layer F.Cu) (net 6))
 (segment (start 123.425 107.08) (end 124.625 105.88) (width 0.15) (layer F.Cu) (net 6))
 (segment (start 124.274999 107.929999) (end 123.425 107.08) (width 0.15) (layer F.Cu) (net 6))
 (segment (start 124.575001 111.129999) (end 124.575001 108.230001) (width 0.15) (layer F.Cu) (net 6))
 (segment (start 124.575001 108.230001) (end 124.274999 107.929999) (width 0.15) (layer F.Cu) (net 6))
 (segment (start 121.795 113.91) (end 124.575001 111.129999) (width 0.15) (layer F.Cu) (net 6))
 (segment (start 117.85 98.17) (end 117.325 98.17) (width 0.15) (layer F.Cu) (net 5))
 (segment (start 120.885 109.62) (end 119.734999 108.469999) (width 0.15) (layer F.Cu) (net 5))
 (segment (start 119.734999 100.054999) (end 117.85 98.17) (width 0.15) (layer F.Cu) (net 5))
 (segment (start 119.734999 108.469999) (end 119.734999 100.054999) (width 0.15) (layer F.Cu) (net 5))
 (segment (start 120.885 109.62) (end 123.185 111.92) (width 0.15) (layer B.Cu) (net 5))
 (segment (start 149.825 131.73) (end 149.825 134.38) (width 0.15) (layer F.Cu) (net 5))
 (segment (start 148.79 130.695) (end 149.825 131.73) (width 0.15) (layer F.Cu) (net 5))
 (segment (start 149.835 88.17) (end 148.79 89.215) (width 0.15) (layer F.Cu) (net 5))
 (via (at 148.79 111.92) (size 0.8) (drill 0.4) (layers F.Cu B.Cu) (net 5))
 (segment (start 148.79 111.92) (end 148.79 130.695) (width 0.15) (layer F.Cu) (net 5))
 (segment (start 148.79 89.215) (end 148.79 111.92) (width 0.15) (layer F.Cu) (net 5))
 (segment (start 123.185 111.92) (end 148.79 111.92) (width 0.15) (layer B.Cu) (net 5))
 (segment (start 149.779997 108.205001) (end 149.779999 108.204999) (width 0.15) (layer B.Cu) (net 4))
 (segment (start 116.13 101.38) (end 116.8 100.71) (width 0.15) (layer F.Cu) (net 4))
 (segment (start 116.13 109.107002) (end 116.13 101.38) (width 0.15) (layer F.Cu) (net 4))
 (segment (start 117.792999 110.770001) (end 116.13 109.107002) (width 0.15) (layer F.Cu) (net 4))
 (segment (start 116.8 100.71) (end 117.325 100.71) (width 0.15) (layer F.Cu) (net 4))
 (segment (start 122.035001 110.172001) (end 121.437001 110.770001) (width 0.15) (layer F.Cu) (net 4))
 (segment (start 122.035001 108.230001) (end 122.035001 110.172001) (width 0.15) (layer F.Cu) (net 4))
 (segment (start 121.437001 110.770001) (end 117.792999 110.770001) (width 0.15) (layer F.Cu) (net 4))
 (segment (start 120.885 107.08) (end 122.035001 108.230001) (width 0.15) (layer F.Cu) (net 4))
 (segment (start 152.365 132.63) (end 152.365 134.38) (width 0.15) (layer F.Cu) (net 4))
 (segment (start 149.49 129.755) (end 152.365 132.63) (width 0.15) (layer F.Cu) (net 4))
 (segment (start 152.375 88.17) (end 149.49 91.055) (width 0.15) (layer F.Cu) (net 4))
 (segment (start 120.885 107.08) (end 122.275 108.47) (width 0.15) (layer B.Cu) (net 4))
 (segment (start 149.49 108.47) (end 149.49 129.755) (width 0.15) (layer F.Cu) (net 4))
 (via (at 149.49 108.47) (size 0.8) (drill 0.4) (layers F.Cu B.Cu) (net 4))
 (segment (start 149.49 91.055) (end 149.49 108.47) (width 0.15) (layer F.Cu) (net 4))
 (segment (start 122.275 108.47) (end 149.49 108.47) (width 0.15) (layer B.Cu) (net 4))
 (segment (start 117.85 99.44) (end 117.325 99.44) (width 0.15) (layer F.Cu) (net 7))
 (segment (start 118.345 107.08) (end 118.345 106.03) (width 0.15) (layer F.Cu) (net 7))
 (segment (start 118.345 106.03) (end 118.475001 105.899999) (width 0.15) (layer F.Cu) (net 7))
 (segment (start 118.475001 105.899999) (end 118.475001 100.065001) (width 0.15) (layer F.Cu) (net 7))
 (segment (start 118.475001 100.065001) (end 117.85 99.44) (width 0.15) (layer F.Cu) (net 7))
 (segment (start 176.485 96.175) (end 175.76 95.45) (width 0.2) (layer F.Cu) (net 9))
 (segment (start 176.485 99.56) (end 176.485 96.175) (width 0.2) (layer F.Cu) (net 9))
 (via (at 172.875 100.67) (size 0.8) (drill 0.4) (layers F.Cu B.Cu) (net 8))
 (segment (start 174.185 99.36) (end 172.875 100.67) (width 0.15) (layer F.Cu) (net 8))
 (segment (start 174.185 95.45) (end 174.185 99.36) (width 0.15) (layer F.Cu) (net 8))
 (via (at 126.67 100.67) (size 0.8) (drill 0.4) (layers F.Cu B.Cu) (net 8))
 (segment (start 172.875 100.67) (end 126.67 100.67) (width 0.15) (layer B.Cu) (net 8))
 (segment (start 124.665 100.67) (end 124.625 100.71) (width 0.15) (layer F.Cu) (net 8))
 (segment (start 126.67 100.67) (end 124.665 100.67) (width 0.15) (layer F.Cu) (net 8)))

